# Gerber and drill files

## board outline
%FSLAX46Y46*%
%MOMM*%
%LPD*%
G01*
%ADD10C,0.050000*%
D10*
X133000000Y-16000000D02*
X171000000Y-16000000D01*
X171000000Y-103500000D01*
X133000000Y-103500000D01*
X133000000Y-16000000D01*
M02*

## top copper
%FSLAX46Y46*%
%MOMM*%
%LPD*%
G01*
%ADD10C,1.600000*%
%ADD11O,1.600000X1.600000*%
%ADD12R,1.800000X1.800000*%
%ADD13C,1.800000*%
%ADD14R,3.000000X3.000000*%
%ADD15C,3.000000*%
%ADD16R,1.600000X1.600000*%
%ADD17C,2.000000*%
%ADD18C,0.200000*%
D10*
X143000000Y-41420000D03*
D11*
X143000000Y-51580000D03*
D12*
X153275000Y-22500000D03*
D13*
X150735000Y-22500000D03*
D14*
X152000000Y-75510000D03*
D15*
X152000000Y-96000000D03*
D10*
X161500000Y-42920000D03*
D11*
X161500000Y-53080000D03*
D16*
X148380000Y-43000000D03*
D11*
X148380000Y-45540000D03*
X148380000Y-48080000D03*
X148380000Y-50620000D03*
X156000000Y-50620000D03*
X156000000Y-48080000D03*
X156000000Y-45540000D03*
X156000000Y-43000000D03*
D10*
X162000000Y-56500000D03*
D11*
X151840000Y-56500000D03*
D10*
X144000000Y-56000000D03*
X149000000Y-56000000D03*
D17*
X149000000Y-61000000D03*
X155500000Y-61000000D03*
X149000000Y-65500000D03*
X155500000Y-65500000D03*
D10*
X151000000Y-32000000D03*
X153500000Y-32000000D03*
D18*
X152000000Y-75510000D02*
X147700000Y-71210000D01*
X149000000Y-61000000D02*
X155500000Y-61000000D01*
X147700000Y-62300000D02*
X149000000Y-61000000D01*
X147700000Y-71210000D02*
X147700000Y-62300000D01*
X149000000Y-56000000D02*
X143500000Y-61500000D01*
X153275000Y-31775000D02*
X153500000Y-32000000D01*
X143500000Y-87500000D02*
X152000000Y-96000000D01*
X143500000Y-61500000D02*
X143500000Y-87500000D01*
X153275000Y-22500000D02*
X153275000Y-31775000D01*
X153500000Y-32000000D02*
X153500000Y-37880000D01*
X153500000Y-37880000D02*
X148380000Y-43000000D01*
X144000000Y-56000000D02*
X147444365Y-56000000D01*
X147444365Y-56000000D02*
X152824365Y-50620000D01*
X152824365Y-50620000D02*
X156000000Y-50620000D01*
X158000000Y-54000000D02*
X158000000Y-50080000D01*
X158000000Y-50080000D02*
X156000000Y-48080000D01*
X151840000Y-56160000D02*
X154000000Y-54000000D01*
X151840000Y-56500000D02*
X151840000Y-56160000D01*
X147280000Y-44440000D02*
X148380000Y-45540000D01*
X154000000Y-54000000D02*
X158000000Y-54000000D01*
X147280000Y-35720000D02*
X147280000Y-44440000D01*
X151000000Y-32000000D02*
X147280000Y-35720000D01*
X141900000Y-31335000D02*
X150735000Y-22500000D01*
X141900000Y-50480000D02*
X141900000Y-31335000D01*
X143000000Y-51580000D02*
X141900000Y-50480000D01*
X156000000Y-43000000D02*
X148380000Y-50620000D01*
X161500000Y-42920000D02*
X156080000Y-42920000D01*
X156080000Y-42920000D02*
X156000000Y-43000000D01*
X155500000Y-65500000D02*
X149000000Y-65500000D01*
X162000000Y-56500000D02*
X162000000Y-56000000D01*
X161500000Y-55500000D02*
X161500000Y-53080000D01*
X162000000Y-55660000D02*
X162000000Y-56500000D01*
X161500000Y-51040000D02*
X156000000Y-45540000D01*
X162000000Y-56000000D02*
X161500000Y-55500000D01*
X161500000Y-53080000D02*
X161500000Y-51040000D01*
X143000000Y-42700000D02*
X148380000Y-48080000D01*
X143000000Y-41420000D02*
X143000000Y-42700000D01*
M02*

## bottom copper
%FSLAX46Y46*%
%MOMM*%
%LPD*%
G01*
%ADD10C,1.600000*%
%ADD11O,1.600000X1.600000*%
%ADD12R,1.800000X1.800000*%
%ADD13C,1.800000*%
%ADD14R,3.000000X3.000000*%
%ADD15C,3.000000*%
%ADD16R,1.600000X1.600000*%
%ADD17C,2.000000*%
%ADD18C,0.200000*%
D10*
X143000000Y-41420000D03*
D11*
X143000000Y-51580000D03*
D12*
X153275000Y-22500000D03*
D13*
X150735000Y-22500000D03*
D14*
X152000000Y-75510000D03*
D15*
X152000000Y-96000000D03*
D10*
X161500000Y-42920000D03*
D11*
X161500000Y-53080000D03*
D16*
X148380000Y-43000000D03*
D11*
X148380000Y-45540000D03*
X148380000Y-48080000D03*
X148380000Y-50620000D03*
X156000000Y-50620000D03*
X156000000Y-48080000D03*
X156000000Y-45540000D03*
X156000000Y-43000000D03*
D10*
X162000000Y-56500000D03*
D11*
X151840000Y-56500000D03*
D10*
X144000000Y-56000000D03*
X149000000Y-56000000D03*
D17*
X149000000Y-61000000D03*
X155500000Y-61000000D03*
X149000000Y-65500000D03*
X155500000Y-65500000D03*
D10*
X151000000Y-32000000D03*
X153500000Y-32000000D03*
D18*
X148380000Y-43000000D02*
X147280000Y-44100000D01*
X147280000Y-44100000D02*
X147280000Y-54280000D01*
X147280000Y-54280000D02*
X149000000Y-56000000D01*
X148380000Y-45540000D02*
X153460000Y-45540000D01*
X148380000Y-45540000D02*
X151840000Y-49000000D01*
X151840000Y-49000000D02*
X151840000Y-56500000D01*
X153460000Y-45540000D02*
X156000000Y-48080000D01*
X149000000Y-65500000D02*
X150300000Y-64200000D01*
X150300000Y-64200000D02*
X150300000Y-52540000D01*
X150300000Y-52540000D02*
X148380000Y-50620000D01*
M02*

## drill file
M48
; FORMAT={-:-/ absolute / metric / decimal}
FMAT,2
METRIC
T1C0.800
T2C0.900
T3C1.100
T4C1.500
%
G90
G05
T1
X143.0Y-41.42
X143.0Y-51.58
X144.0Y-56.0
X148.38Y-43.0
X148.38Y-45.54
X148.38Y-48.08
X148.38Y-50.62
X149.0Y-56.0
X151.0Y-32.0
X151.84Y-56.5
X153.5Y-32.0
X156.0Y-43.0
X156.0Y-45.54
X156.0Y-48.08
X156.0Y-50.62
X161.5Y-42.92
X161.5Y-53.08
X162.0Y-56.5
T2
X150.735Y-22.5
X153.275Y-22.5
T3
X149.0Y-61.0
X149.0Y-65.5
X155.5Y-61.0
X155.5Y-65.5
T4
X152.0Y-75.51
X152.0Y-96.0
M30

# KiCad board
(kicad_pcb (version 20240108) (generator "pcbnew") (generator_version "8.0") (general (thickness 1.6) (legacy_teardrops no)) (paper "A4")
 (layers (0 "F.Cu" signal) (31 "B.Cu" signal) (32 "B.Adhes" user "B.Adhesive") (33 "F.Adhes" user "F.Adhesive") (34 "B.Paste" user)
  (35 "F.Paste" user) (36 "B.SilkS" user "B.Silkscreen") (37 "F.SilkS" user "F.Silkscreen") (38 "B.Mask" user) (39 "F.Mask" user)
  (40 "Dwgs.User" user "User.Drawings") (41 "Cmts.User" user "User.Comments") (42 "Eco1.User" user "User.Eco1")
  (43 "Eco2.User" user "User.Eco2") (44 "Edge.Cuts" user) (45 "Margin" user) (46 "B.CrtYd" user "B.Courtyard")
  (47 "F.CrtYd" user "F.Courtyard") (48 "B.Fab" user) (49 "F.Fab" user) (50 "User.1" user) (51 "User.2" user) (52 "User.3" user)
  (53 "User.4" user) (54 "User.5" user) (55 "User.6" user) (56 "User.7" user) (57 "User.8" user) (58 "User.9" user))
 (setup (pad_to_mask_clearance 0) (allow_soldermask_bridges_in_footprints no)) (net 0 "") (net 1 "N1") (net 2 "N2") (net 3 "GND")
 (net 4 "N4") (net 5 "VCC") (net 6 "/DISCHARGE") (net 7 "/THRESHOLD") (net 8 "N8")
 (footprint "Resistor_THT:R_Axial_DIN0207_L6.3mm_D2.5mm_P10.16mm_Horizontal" (layer "F.Cu") (at 143 41.42 -90)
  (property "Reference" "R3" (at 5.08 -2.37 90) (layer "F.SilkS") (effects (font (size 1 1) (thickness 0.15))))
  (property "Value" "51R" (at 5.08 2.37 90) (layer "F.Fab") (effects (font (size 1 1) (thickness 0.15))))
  (pad "1" thru_hole circle (at 0 0 270) (size 1.6 1.6) (drill 0.8) (layers "*.Cu" "*.Mask") (remove_unused_layers no) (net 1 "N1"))
  (pad "2" thru_hole oval (at 10.16 0 270) (size 1.6 1.6) (drill 0.8) (layers "*.Cu" "*.Mask") (remove_unused_layers no) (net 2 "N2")))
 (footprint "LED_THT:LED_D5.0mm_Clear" (layer "F.Cu") (at 153.275 22.5 180)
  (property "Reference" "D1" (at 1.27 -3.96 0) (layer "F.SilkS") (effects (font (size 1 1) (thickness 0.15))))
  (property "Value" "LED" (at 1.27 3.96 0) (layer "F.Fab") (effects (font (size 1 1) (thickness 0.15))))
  (pad "1" thru_hole rect (at 0 0 180) (size 1.8 1.8) (drill 0.9) (layers "*.Cu" "*.Mask") (remove_unused_layers no) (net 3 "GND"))
  (pad "2" thru_hole circle (at 2.54 0 180) (size 1.8 1.8) (drill 0.9) (layers "*.Cu" "*.Mask") (remove_unused_layers no) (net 2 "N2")))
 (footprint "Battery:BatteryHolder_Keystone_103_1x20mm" (layer "F.Cu") (at 152 75.51 -90)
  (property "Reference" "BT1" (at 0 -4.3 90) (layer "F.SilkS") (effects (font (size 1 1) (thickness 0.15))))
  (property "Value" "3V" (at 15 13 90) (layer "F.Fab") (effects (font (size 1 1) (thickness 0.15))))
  (pad "1" thru_hole rect (at 0 0 270) (size 3 3) (drill 1.5) (layers "*.Cu" "*.Mask") (remove_unused_layers no) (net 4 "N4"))
  (pad "2" thru_hole circle (at 20.49 0 270) (size 3 3) (drill 1.5) (layers "*.Cu" "*.Mask") (remove_unused_layers no) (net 3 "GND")))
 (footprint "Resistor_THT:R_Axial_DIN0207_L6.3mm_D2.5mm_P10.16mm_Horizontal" (layer "F.Cu") (at 161.5 42.92 -90)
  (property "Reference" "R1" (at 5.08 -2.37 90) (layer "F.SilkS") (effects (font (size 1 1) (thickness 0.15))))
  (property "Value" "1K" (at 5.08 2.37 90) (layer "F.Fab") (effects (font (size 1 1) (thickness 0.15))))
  (pad "1" thru_hole circle (at 0 0 270) (size 1.6 1.6) (drill 0.8) (layers "*.Cu" "*.Mask") (remove_unused_layers no) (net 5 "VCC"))
  (pad "2" thru_hole oval (at 10.16 0 270) (size 1.6 1.6) (drill 0.8) (layers "*.Cu" "*.Mask") (remove_unused_layers no)
   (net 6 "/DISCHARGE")))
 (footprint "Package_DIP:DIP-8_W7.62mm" (layer "F.Cu") (at 148.38 43)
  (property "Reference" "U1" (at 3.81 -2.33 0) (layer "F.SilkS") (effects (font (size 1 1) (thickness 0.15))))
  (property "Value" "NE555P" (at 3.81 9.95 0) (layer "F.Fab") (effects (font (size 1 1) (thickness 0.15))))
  (pad "1" thru_hole rect (at 0 0) (size 1.6 1.6) (drill 0.8) (layers "*.Cu" "*.Mask") (remove_unused_layers no) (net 3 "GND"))
  (pad "2" thru_hole oval (at 0 2.54) (size 1.6 1.6) (drill 0.8) (layers "*.Cu" "*.Mask") (remove_unused_layers no) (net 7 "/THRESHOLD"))
  (pad "3" thru_hole oval (at 0 5.08) (size 1.6 1.6) (drill 0.8) (layers "*.Cu" "*.Mask") (remove_unused_layers no) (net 1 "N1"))
  (pad "4" thru_hole oval (at 0 7.62) (size 1.6 1.6) (drill 0.8) (layers "*.Cu" "*.Mask") (remove_unused_layers no) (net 5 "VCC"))
  (pad "5" thru_hole oval (at 7.62 7.62) (size 1.6 1.6) (drill 0.8) (layers "*.Cu" "*.Mask") (remove_unused_layers no) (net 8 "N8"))
  (pad "6" thru_hole oval (at 7.62 5.08) (size 1.6 1.6) (drill 0.8) (layers "*.Cu" "*.Mask") (remove_unused_layers no) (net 7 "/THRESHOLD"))
  (pad "7" thru_hole oval (at 7.62 2.54) (size 1.6 1.6) (drill 0.8) (layers "*.Cu" "*.Mask") (remove_unused_layers no) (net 6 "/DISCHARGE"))
  (pad "8" thru_hole oval (at 7.62 0) (size 1.6 1.6) (drill 0.8) (layers "*.Cu" "*.Mask") (remove_unused_layers no) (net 5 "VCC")))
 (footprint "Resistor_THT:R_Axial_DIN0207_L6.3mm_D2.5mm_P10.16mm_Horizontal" (layer "F.Cu") (at 162 56.5 180)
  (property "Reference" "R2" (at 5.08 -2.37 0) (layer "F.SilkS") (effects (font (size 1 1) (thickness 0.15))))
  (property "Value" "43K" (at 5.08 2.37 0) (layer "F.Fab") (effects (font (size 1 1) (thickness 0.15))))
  (pad "1" thru_hole circle (at 0 0 180) (size 1.6 1.6) (drill 0.8) (layers "*.Cu" "*.Mask") (remove_unused_layers no) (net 6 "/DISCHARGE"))
  (pad "2" thru_hole oval (at 10.16 0 180) (size 1.6 1.6) (drill 0.8) (layers "*.Cu" "*.Mask") (remove_unused_layers no)
   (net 7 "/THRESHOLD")))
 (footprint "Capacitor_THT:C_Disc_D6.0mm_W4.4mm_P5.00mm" (layer "F.Cu") (at 144 56)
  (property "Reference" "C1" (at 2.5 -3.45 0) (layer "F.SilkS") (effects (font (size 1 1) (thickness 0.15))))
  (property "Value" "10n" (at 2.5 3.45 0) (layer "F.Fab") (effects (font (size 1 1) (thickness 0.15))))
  (pad "1" thru_hole circle (at 0 0) (size 1.6 1.6) (drill 0.8) (layers "*.Cu" "*.Mask") (remove_unused_layers no) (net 8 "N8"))
  (pad "2" thru_hole circle (at 5 0) (size 1.6 1.6) (drill 0.8) (layers "*.Cu" "*.Mask") (remove_unused_layers no) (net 3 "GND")))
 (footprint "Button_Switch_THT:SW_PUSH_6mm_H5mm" (layer "F.Cu") (at 149 61)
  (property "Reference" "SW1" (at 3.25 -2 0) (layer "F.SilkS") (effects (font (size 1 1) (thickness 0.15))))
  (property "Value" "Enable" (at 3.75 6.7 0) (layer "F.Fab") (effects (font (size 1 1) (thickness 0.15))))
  (pad "1" thru_hole circle (at 0 0 90) (size 2 2) (drill 1.1) (layers "*.Cu" "*.Mask") (remove_unused_layers no) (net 4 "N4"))
  (pad "1" thru_hole circle (at 6.5 0 90) (size 2 2) (drill 1.1) (layers "*.Cu" "*.Mask") (remove_unused_layers no) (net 4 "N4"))
  (pad "2" thru_hole circle (at 0 4.5 90) (size 2 2) (drill 1.1) (layers "*.Cu" "*.Mask") (remove_unused_layers no) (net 5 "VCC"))
  (pad "2" thru_hole circle (at 6.5 4.5 90) (size 2 2) (drill 1.1) (layers "*.Cu" "*.Mask") (remove_unused_layers no) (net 5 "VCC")))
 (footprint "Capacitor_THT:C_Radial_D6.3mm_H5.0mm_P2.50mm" (layer "F.Cu") (at 151 32)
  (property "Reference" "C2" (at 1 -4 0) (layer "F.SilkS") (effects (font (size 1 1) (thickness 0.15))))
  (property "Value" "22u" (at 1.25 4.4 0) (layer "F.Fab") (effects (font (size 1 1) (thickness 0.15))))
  (pad "1" thru_hole circle (at 0 0) (size 1.6 1.6) (drill 0.8) (layers "*.Cu" "*.Mask") (remove_unused_layers no) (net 7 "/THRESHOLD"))
  (pad "2" thru_hole circle (at 2.5 0) (size 1.6 1.6) (drill 0.8) (layers "*.Cu" "*.Mask") (remove_unused_layers no) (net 3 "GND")))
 (gr_rect (start 133 16) (end 171 103.5) (stroke (width 0.05) (type default)) (fill none) (layer "Edge.Cuts"))
 (segment (start 152 75.51) (end 147.7 71.21) (width 0.2) (layer "F.Cu") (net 4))
 (segment (start 149 61) (end 155.5 61) (width 0.2) (layer "F.Cu") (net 4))
 (segment (start 147.7 62.3) (end 149 61) (width 0.2) (layer "F.Cu") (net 4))
 (segment (start 147.7 71.21) (end 147.7 62.3) (width 0.2) (layer "F.Cu") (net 4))
 (segment (start 149 56) (end 143.5 61.5) (width 0.2) (layer "F.Cu") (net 3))
 (segment (start 153.275 31.775) (end 153.5 32) (width 0.2) (layer "F.Cu") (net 3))
 (segment (start 143.5 87.5) (end 152 96) (width 0.2) (layer "F.Cu") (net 3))
 (segment (start 143.5 61.5) (end 143.5 87.5) (width 0.2) (layer "F.Cu") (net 3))
 (segment (start 153.275 22.5) (end 153.275 31.775) (width 0.2) (layer "F.Cu") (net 3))
 (segment (start 153.5 32) (end 153.5 37.88) (width 0.2) (layer "F.Cu") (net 3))
 (segment (start 153.5 37.88) (end 148.38 43) (width 0.2) (layer "F.Cu") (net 3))
 (segment (start 148.38 43) (end 147.28 44.1) (width 0.2) (layer "B.Cu") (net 3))
 (segment (start 147.28 44.1) (end 147.28 54.28) (width 0.2) (layer "B.Cu") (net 3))
 (segment (start 147.28 54.28) (end 149 56) (width 0.2) (layer "B.Cu") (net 3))
 (segment (start 144 56) (end 147.444365 56) (width 0.2) (layer "F.Cu") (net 8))
 (segment (start 147.444365 56) (end 152.824365 50.62) (width 0.2) (layer "F.Cu") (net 8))
 (segment (start 152.824365 50.62) (end 156 50.62) (width 0.2) (layer "F.Cu") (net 8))
 (segment (start 158 54) (end 158 50.08) (width 0.2) (layer "F.Cu") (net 7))
 (segment (start 158 50.08) (end 156 48.08) (width 0.2) (layer "F.Cu") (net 7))
 (segment (start 151.84 56.16) (end 154 54) (width 0.2) (layer "F.Cu") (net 7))
 (segment (start 151.84 56.5) (end 151.84 56.16) (width 0.2) (layer "F.Cu") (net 7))
 (segment (start 147.28 44.44) (end 148.38 45.54) (width 0.2) (layer "F.Cu") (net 7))
 (segment (start 154 54) (end 158 54) (width 0.2) (layer "F.Cu") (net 7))
 (segment (start 147.28 35.72) (end 147.28 44.44) (width 0.2) (layer "F.Cu") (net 7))
 (segment (start 151 32) (end 147.28 35.72) (width 0.2) (layer "F.Cu") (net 7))
 (segment (start 148.38 45.54) (end 153.46 45.54) (width 0.2) (layer "B.Cu") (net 7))
 (segment (start 148.38 45.54) (end 151.84 49) (width 0.2) (layer "B.Cu") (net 7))
 (segment (start 151.84 49) (end 151.84 56.5) (width 0.2) (layer "B.Cu") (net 7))
 (segment (start 153.46 45.54) (end 156 48.08) (width 0.2) (layer "B.Cu") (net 7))
 (segment (start 141.9 31.335) (end 150.735 22.5) (width 0.2) (layer "F.Cu") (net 2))
 (segment (start 141.9 50.48) (end 141.9 31.335) (width 0.2) (layer "F.Cu") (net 2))
 (segment (start 143 51.58) (end 141.9 50.48) (width 0.2) (layer "F.Cu") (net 2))
 (segment (start 156 43) (end 148.38 50.62) (width 0.2) (layer "F.Cu") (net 5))
 (segment (start 161.5 42.92) (end 156.08 42.92) (width 0.2) (layer "F.Cu") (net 5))
 (segment (start 156.08 42.92) (end 156 43) (width 0.2) (layer "F.Cu") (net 5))
 (segment (start 155.5 65.5) (end 149 65.5) (width 0.2) (layer "F.Cu") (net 5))
 (segment (start 149 65.5) (end 150.3 64.2) (width 0.2) (layer "B.Cu") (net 5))
 (segment (start 150.3 64.2) (end 150.3 52.54) (width 0.2) (layer "B.Cu") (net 5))
 (segment (start 150.3 52.54) (end 148.38 50.62) (width 0.2) (layer "B.Cu") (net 5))
 (segment (start 162 56.5) (end 162 56) (width 0.2) (layer "F.Cu") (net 6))
 (segment (start 161.5 55.5) (end 161.5 53.08) (width 0.2) (layer "F.Cu") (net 6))
 (segment (start 162 55.66) (end 162 56.5) (width 0.2) (layer "F.Cu") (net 6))
 (segment (start 161.5 51.04) (end 156 45.54) (width 0.2) (layer "F.Cu") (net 6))
 (segment (start 162 56) (end 161.5 55.5) (width 0.2) (layer "F.Cu") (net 6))
 (segment (start 161.5 53.08) (end 161.5 51.04) (width 0.2) (layer "F.Cu") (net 6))
 (segment (start 143 42.7) (end 148.38 48.08) (width 0.2) (layer "F.Cu") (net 1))
 (segment (start 143 41.42) (end 143 42.7) (width 0.2) (layer "F.Cu") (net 1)))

